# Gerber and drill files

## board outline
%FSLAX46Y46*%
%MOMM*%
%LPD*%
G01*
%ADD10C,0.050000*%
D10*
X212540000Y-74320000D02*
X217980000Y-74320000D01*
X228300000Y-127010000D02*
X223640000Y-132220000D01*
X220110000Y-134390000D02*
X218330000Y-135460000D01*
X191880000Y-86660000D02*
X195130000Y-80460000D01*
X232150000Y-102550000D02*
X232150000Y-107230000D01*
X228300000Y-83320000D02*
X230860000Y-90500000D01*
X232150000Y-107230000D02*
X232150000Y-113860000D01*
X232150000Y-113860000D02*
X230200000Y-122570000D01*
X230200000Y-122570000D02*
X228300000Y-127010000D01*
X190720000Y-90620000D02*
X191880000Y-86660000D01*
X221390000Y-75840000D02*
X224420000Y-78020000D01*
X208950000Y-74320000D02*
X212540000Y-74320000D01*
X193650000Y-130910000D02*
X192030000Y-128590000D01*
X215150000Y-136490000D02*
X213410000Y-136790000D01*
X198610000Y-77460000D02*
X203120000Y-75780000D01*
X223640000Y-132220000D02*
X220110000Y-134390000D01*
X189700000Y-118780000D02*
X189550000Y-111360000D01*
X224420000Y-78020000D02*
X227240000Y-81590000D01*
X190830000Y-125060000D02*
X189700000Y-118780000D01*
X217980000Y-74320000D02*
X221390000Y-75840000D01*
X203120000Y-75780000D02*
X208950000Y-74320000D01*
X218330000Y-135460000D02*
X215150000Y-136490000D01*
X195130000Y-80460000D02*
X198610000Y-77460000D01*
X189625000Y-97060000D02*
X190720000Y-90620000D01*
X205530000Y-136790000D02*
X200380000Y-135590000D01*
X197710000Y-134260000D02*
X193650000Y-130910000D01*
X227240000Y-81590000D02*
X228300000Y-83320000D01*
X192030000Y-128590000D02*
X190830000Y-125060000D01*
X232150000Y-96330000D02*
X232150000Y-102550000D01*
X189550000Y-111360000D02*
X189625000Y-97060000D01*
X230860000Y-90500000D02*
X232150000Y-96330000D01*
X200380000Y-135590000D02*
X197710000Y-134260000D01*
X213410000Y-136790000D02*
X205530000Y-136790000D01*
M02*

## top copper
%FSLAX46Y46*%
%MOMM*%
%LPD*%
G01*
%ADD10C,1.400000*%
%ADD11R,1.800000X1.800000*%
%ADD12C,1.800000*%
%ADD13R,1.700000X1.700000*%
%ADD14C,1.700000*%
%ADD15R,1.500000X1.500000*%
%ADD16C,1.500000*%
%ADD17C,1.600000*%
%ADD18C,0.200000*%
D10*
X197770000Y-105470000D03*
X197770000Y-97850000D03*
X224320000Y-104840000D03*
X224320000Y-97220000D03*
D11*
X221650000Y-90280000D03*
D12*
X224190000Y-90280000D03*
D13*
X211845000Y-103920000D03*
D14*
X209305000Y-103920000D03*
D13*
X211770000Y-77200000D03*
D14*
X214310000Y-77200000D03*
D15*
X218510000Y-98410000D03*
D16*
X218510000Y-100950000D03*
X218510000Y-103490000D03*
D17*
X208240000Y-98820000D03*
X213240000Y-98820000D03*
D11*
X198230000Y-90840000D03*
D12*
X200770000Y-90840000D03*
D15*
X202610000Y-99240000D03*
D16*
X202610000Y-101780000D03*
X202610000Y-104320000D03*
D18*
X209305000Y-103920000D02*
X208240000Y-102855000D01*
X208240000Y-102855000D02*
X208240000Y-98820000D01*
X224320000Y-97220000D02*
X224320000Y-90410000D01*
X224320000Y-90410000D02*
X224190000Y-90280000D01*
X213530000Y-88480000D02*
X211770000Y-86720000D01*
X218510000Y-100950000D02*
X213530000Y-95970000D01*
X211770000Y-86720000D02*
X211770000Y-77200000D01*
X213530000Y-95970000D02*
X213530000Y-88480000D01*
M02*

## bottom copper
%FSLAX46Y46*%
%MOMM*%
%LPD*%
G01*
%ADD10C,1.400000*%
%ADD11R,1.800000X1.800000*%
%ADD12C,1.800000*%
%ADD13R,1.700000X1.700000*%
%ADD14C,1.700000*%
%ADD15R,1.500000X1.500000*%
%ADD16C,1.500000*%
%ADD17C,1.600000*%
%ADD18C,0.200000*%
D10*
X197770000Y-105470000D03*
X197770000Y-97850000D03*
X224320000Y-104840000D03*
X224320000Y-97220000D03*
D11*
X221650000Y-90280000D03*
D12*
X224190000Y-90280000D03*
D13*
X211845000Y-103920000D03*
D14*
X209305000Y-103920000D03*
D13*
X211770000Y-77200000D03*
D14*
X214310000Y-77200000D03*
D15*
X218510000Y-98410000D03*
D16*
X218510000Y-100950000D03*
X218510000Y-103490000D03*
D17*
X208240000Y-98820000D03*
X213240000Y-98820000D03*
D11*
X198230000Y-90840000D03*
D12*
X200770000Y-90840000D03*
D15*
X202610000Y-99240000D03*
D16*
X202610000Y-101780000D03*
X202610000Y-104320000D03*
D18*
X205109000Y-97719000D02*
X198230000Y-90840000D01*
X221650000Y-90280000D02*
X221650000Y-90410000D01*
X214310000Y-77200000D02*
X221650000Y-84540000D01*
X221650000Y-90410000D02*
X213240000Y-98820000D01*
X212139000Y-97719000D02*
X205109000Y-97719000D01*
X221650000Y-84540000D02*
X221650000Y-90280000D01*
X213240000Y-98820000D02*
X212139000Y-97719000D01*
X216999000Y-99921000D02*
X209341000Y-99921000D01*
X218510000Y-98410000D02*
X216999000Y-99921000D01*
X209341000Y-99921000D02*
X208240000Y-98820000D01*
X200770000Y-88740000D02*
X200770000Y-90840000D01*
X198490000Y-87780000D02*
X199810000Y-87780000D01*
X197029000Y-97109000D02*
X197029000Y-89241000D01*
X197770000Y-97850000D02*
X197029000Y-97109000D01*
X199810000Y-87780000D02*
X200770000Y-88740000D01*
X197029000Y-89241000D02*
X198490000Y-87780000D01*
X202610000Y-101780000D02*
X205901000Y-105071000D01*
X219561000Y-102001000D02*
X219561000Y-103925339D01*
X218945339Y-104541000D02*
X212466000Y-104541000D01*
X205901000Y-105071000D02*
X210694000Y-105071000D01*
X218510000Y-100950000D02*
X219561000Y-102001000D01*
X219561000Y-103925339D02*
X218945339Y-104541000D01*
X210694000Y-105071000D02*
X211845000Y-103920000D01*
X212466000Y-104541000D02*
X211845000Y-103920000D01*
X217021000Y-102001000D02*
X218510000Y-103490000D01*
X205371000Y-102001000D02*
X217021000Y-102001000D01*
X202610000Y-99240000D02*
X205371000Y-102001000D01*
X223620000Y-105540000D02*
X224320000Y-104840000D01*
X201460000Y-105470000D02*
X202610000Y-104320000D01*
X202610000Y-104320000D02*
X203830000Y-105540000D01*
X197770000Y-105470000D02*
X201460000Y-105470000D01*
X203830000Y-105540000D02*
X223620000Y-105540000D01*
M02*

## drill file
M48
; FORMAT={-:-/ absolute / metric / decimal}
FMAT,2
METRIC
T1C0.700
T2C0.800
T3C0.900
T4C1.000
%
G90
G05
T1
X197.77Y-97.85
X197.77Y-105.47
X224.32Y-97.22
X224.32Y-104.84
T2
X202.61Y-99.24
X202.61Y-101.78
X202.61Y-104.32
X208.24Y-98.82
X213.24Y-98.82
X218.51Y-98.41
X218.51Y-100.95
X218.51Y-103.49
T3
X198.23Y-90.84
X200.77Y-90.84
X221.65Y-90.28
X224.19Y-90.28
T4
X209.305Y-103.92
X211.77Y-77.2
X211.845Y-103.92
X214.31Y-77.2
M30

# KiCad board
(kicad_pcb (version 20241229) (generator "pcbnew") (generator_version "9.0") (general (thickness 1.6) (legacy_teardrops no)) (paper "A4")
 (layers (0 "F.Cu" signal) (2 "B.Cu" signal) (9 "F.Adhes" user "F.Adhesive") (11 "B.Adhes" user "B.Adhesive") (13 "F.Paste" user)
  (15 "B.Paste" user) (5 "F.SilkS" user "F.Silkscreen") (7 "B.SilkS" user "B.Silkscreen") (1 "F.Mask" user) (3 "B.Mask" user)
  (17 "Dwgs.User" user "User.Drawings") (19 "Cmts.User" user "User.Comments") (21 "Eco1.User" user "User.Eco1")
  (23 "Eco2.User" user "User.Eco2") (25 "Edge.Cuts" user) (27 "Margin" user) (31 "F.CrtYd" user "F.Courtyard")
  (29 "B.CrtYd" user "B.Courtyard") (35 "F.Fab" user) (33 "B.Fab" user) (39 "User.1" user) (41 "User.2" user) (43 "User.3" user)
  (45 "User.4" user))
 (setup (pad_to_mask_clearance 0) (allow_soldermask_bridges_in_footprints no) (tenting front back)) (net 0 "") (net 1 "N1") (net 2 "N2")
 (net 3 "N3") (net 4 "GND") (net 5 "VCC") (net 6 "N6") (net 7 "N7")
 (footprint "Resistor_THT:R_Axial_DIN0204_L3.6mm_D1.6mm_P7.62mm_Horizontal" (layer "F.Cu") (at 197.77 105.47 90)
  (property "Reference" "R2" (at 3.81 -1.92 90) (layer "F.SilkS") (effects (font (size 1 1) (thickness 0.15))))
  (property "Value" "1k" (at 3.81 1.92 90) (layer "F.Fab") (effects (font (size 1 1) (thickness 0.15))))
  (pad "1" thru_hole circle (at 0 0 90) (size 1.4 1.4) (drill 0.7) (layers "*.Cu" "*.Mask") (remove_unused_layers no) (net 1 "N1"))
  (pad "2" thru_hole circle (at 7.62 0 90) (size 1.4 1.4) (drill 0.7) (layers "*.Cu" "*.Mask") (remove_unused_layers no) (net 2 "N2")))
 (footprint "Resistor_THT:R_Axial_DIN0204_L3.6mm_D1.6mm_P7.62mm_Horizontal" (layer "F.Cu") (at 224.32 104.84 90)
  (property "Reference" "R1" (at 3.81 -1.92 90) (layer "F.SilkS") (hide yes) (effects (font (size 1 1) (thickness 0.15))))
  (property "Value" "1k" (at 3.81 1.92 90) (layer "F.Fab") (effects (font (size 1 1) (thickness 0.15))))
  (pad "1" thru_hole circle (at 0 0 90) (size 1.4 1.4) (drill 0.7) (layers "*.Cu" "*.Mask") (remove_unused_layers no) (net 1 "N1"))
  (pad "2" thru_hole circle (at 7.62 0 90) (size 1.4 1.4) (drill 0.7) (layers "*.Cu" "*.Mask") (remove_unused_layers no) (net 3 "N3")))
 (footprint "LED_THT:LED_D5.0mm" (layer "F.Cu") (at 221.65 90.28)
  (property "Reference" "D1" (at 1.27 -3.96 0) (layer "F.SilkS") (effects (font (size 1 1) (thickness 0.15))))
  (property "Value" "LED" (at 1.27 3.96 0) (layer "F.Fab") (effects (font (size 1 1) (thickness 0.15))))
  (pad "1" thru_hole rect (at 0 0) (size 1.8 1.8) (drill 0.9) (layers "*.Cu" "*.Mask") (remove_unused_layers no) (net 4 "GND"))
  (pad "2" thru_hole circle (at 2.54 0) (size 1.8 1.8) (drill 0.9) (layers "*.Cu" "*.Mask") (remove_unused_layers no) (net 3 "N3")))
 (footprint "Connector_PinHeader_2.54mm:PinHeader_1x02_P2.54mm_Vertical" (layer "F.Cu") (at 211.845 103.92 -90)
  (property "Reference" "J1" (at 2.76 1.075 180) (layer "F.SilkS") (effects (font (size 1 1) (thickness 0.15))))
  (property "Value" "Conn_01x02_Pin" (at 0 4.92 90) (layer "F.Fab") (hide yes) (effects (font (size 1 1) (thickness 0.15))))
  (pad "1" thru_hole rect (at 0 0 270) (size 1.7 1.7) (drill 1) (layers "*.Cu" "*.Mask") (remove_unused_layers no) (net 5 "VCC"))
  (pad "2" thru_hole circle (at 0 2.54 270) (size 1.7 1.7) (drill 1) (layers "*.Cu" "*.Mask") (remove_unused_layers no) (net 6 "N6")))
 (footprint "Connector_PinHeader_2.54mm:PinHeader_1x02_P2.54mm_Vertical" (layer "F.Cu") (at 211.77 77.2 90)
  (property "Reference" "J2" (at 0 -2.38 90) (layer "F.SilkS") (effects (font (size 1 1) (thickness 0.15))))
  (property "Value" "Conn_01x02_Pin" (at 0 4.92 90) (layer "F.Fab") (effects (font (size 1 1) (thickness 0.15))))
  (pad "1" thru_hole rect (at 0 0 90) (size 1.7 1.7) (drill 1) (layers "*.Cu" "*.Mask") (remove_unused_layers no) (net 5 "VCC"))
  (pad "2" thru_hole circle (at 0 2.54 90) (size 1.7 1.7) (drill 1) (layers "*.Cu" "*.Mask") (remove_unused_layers no) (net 4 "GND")))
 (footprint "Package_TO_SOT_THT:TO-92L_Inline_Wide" (layer "F.Cu") (at 218.51 98.41 -90)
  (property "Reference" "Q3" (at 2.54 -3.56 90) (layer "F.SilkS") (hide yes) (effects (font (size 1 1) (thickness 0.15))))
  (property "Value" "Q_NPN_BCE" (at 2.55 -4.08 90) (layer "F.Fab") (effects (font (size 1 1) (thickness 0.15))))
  (pad "1" thru_hole rect (at 0 0 270) (size 1.5 1.5) (drill 0.8) (layers "*.Cu" "*.Mask") (remove_unused_layers no) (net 6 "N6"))
  (pad "2" thru_hole circle (at 2.54 0 270) (size 1.5 1.5) (drill 0.8) (layers "*.Cu" "*.Mask") (remove_unused_layers no) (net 5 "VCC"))
  (pad "3" thru_hole circle (at 5.08 0 270) (size 1.5 1.5) (drill 0.8) (layers "*.Cu" "*.Mask") (remove_unused_layers no) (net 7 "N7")))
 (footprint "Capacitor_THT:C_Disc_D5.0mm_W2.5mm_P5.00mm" (layer "F.Cu") (at 208.24 98.82)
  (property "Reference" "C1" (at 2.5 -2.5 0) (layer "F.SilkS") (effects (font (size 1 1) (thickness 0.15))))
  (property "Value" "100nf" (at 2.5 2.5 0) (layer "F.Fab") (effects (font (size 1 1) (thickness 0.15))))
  (pad "1" thru_hole circle (at 0 0) (size 1.6 1.6) (drill 0.8) (layers "*.Cu" "*.Mask") (remove_unused_layers no) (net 6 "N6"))
  (pad "2" thru_hole circle (at 5 0) (size 1.6 1.6) (drill 0.8) (layers "*.Cu" "*.Mask") (remove_unused_layers no) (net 4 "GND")))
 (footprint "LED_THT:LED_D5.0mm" (layer "F.Cu") (at 198.23 90.84)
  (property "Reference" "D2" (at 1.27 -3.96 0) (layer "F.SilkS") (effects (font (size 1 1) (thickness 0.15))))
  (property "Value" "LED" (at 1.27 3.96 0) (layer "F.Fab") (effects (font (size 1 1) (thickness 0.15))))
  (pad "1" thru_hole rect (at 0 0) (size 1.8 1.8) (drill 0.9) (layers "*.Cu" "*.Mask") (remove_unused_layers no) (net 4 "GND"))
  (pad "2" thru_hole circle (at 2.54 0) (size 1.8 1.8) (drill 0.9) (layers "*.Cu" "*.Mask") (remove_unused_layers no) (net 2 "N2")))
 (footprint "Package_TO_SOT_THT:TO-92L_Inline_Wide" (layer "F.Cu") (at 202.61 99.24 -90)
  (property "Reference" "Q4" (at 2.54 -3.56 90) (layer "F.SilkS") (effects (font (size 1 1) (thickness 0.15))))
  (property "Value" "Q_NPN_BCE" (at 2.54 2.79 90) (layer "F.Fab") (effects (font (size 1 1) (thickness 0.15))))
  (pad "1" thru_hole rect (at 0 0 270) (size 1.5 1.5) (drill 0.8) (layers "*.Cu" "*.Mask") (remove_unused_layers no) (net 7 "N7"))
  (pad "2" thru_hole circle (at 2.54 0 270) (size 1.5 1.5) (drill 0.8) (layers "*.Cu" "*.Mask") (remove_unused_layers no) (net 5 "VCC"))
  (pad "3" thru_hole circle (at 5.08 0 270) (size 1.5 1.5) (drill 0.8) (layers "*.Cu" "*.Mask") (remove_unused_layers no) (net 1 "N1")))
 (gr_line (start 212.54 74.32) (end 217.98 74.32) (stroke (width 0.05) (type default)) (layer "Edge.Cuts"))
 (gr_line (start 228.3 127.01) (end 223.64 132.22) (stroke (width 0.05) (type default)) (layer "Edge.Cuts"))
 (gr_line (start 220.11 134.39) (end 218.33 135.46) (stroke (width 0.05) (type default)) (layer "Edge.Cuts"))
 (gr_line (start 191.88 86.66) (end 195.13 80.46) (stroke (width 0.05) (type default)) (layer "Edge.Cuts"))
 (gr_line (start 232.15 102.55) (end 232.15 107.23) (stroke (width 0.05) (type default)) (layer "Edge.Cuts"))
 (gr_line (start 228.3 83.32) (end 230.86 90.5) (stroke (width 0.05) (type default)) (layer "Edge.Cuts"))
 (gr_line (start 232.15 107.23) (end 232.15 113.86) (stroke (width 0.05) (type default)) (layer "Edge.Cuts"))
 (gr_line (start 232.15 113.86) (end 230.2 122.57) (stroke (width 0.05) (type default)) (layer "Edge.Cuts"))
 (gr_line (start 230.2 122.57) (end 228.3 127.01) (stroke (width 0.05) (type default)) (layer "Edge.Cuts"))
 (gr_line (start 190.72 90.62) (end 191.88 86.66) (stroke (width 0.05) (type default)) (layer "Edge.Cuts"))
 (gr_line (start 221.39 75.84) (end 224.42 78.02) (stroke (width 0.05) (type default)) (layer "Edge.Cuts"))
 (gr_line (start 208.95 74.32) (end 212.54 74.32) (stroke (width 0.05) (type default)) (layer "Edge.Cuts"))
 (gr_line (start 193.65 130.91) (end 192.03 128.59) (stroke (width 0.05) (type default)) (layer "Edge.Cuts"))
 (gr_line (start 215.15 136.49) (end 213.41 136.79) (stroke (width 0.05) (type default)) (layer "Edge.Cuts"))
 (gr_line (start 198.61 77.46) (end 203.12 75.78) (stroke (width 0.05) (type default)) (layer "Edge.Cuts"))
 (gr_line (start 223.64 132.22) (end 220.11 134.39) (stroke (width 0.05) (type default)) (layer "Edge.Cuts"))
 (gr_line (start 189.7 118.78) (end 189.55 111.36) (stroke (width 0.05) (type default)) (layer "Edge.Cuts"))
 (gr_line (start 224.42 78.02) (end 227.24 81.59) (stroke (width 0.05) (type default)) (layer "Edge.Cuts"))
 (gr_line (start 190.83 125.06) (end 189.7 118.78) (stroke (width 0.05) (type default)) (layer "Edge.Cuts"))
 (gr_line (start 217.98 74.32) (end 221.39 75.84) (stroke (width 0.05) (type default)) (layer "Edge.Cuts"))
 (gr_line (start 203.12 75.78) (end 208.95 74.32) (stroke (width 0.05) (type default)) (layer "Edge.Cuts"))
 (gr_line (start 218.33 135.46) (end 215.15 136.49) (stroke (width 0.05) (type default)) (layer "Edge.Cuts"))
 (gr_line (start 195.13 80.46) (end 198.61 77.46) (stroke (width 0.05) (type default)) (layer "Edge.Cuts"))
 (gr_line (start 189.625 97.06) (end 190.72 90.62) (stroke (width 0.05) (type default)) (layer "Edge.Cuts"))
 (gr_line (start 205.53 136.79) (end 200.38 135.59) (stroke (width 0.05) (type default)) (layer "Edge.Cuts"))
 (gr_line (start 197.71 134.26) (end 193.65 130.91) (stroke (width 0.05) (type default)) (layer "Edge.Cuts"))
 (gr_line (start 227.24 81.59) (end 228.3 83.32) (stroke (width 0.05) (type default)) (layer "Edge.Cuts"))
 (gr_line (start 192.03 128.59) (end 190.83 125.06) (stroke (width 0.05) (type default)) (layer "Edge.Cuts"))
 (gr_line (start 232.15 96.33) (end 232.15 102.55) (stroke (width 0.05) (type default)) (layer "Edge.Cuts"))
 (gr_line (start 189.55 111.36) (end 189.625 97.06) (stroke (width 0.05) (type default)) (layer "Edge.Cuts"))
 (gr_line (start 230.86 90.5) (end 232.15 96.33) (stroke (width 0.05) (type default)) (layer "Edge.Cuts"))
 (gr_line (start 200.38 135.59) (end 197.71 134.26) (stroke (width 0.05) (type default)) (layer "Edge.Cuts"))
 (gr_line (start 213.41 136.79) (end 205.53 136.79) (stroke (width 0.05) (type default)) (layer "Edge.Cuts"))
 (segment (start 205.109 97.719) (end 198.23 90.84) (width 0.2) (layer "B.Cu") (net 4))
 (segment (start 221.65 90.28) (end 221.65 90.41) (width 0.2) (layer "B.Cu") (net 4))
 (segment (start 214.31 77.2) (end 221.65 84.54) (width 0.2) (layer "B.Cu") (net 4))
 (segment (start 221.65 90.41) (end 213.24 98.82) (width 0.2) (layer "B.Cu") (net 4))
 (segment (start 212.139 97.719) (end 205.109 97.719) (width 0.2) (layer "B.Cu") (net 4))
 (segment (start 221.65 84.54) (end 221.65 90.28) (width 0.2) (layer "B.Cu") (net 4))
 (segment (start 213.24 98.82) (end 212.139 97.719) (width 0.2) (layer "B.Cu") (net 4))
 (segment (start 209.305 103.92) (end 208.24 102.855) (width 0.2) (layer "F.Cu") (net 6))
 (segment (start 208.24 102.855) (end 208.24 98.82) (width 0.2) (layer "F.Cu") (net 6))
 (segment (start 216.999 99.921) (end 209.341 99.921) (width 0.2) (layer "B.Cu") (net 6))
 (segment (start 218.51 98.41) (end 216.999 99.921) (width 0.2) (layer "B.Cu") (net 6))
 (segment (start 209.341 99.921) (end 208.24 98.82) (width 0.2) (layer "B.Cu") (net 6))
 (segment (start 224.32 97.22) (end 224.32 90.41) (width 0.2) (layer "F.Cu") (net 3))
 (segment (start 224.32 90.41) (end 224.19 90.28) (width 0.2) (layer "F.Cu") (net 3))
 (segment (start 200.77 88.74) (end 200.77 90.84) (width 0.2) (layer "B.Cu") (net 2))
 (segment (start 198.49 87.78) (end 199.81 87.78) (width 0.2) (layer "B.Cu") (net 2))
 (segment (start 197.029 97.109) (end 197.029 89.241) (width 0.2) (layer "B.Cu") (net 2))
 (segment (start 197.77 97.85) (end 197.029 97.109) (width 0.2) (layer "B.Cu") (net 2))
 (segment (start 199.81 87.78) (end 200.77 88.74) (width 0.2) (layer "B.Cu") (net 2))
 (segment (start 197.029 89.241) (end 198.49 87.78) (width 0.2) (layer "B.Cu") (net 2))
 (segment (start 213.53 88.48) (end 211.77 86.72) (width 0.2) (layer "F.Cu") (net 5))
 (segment (start 218.51 100.95) (end 213.53 95.97) (width 0.2) (layer "F.Cu") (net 5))
 (segment (start 211.77 86.72) (end 211.77 77.2) (width 0.2) (layer "F.Cu") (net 5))
 (segment (start 213.53 95.97) (end 213.53 88.48) (width 0.2) (layer "F.Cu") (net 5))
 (segment (start 202.61 101.78) (end 205.901 105.071) (width 0.2) (layer "B.Cu") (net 5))
 (segment (start 219.561 102.001) (end 219.561 103.925339) (width 0.2) (layer "B.Cu") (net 5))
 (segment (start 218.945339 104.541) (end 212.466 104.541) (width 0.2) (layer "B.Cu") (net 5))
 (segment (start 205.901 105.071) (end 210.694 105.071) (width 0.2) (layer "B.Cu") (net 5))
 (segment (start 218.51 100.95) (end 219.561 102.001) (width 0.2) (layer "B.Cu") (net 5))
 (segment (start 219.561 103.925339) (end 218.945339 104.541) (width 0.2) (layer "B.Cu") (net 5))
 (segment (start 210.694 105.071) (end 211.845 103.92) (width 0.2) (layer "B.Cu") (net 5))
 (segment (start 212.466 104.541) (end 211.845 103.92) (width 0.2) (layer "B.Cu") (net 5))
 (segment (start 217.021 102.001) (end 218.51 103.49) (width 0.2) (layer "B.Cu") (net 7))
 (segment (start 205.371 102.001) (end 217.021 102.001) (width 0.2) (layer "B.Cu") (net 7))
 (segment (start 202.61 99.24) (end 205.371 102.001) (width 0.2) (layer "B.Cu") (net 7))
 (segment (start 223.62 105.54) (end 224.32 104.84) (width 0.2) (layer "B.Cu") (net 1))
 (segment (start 201.46 105.47) (end 202.61 104.32) (width 0.2) (layer "B.Cu") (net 1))
 (segment (start 202.61 104.32) (end 203.83 105.54) (width 0.2) (layer "B.Cu") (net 1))
 (segment (start 197.77 105.47) (end 201.46 105.47) (width 0.2) (layer "B.Cu") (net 1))
 (segment (start 203.83 105.54) (end 223.62 105.54) (width 0.2) (layer "B.Cu") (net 1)))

